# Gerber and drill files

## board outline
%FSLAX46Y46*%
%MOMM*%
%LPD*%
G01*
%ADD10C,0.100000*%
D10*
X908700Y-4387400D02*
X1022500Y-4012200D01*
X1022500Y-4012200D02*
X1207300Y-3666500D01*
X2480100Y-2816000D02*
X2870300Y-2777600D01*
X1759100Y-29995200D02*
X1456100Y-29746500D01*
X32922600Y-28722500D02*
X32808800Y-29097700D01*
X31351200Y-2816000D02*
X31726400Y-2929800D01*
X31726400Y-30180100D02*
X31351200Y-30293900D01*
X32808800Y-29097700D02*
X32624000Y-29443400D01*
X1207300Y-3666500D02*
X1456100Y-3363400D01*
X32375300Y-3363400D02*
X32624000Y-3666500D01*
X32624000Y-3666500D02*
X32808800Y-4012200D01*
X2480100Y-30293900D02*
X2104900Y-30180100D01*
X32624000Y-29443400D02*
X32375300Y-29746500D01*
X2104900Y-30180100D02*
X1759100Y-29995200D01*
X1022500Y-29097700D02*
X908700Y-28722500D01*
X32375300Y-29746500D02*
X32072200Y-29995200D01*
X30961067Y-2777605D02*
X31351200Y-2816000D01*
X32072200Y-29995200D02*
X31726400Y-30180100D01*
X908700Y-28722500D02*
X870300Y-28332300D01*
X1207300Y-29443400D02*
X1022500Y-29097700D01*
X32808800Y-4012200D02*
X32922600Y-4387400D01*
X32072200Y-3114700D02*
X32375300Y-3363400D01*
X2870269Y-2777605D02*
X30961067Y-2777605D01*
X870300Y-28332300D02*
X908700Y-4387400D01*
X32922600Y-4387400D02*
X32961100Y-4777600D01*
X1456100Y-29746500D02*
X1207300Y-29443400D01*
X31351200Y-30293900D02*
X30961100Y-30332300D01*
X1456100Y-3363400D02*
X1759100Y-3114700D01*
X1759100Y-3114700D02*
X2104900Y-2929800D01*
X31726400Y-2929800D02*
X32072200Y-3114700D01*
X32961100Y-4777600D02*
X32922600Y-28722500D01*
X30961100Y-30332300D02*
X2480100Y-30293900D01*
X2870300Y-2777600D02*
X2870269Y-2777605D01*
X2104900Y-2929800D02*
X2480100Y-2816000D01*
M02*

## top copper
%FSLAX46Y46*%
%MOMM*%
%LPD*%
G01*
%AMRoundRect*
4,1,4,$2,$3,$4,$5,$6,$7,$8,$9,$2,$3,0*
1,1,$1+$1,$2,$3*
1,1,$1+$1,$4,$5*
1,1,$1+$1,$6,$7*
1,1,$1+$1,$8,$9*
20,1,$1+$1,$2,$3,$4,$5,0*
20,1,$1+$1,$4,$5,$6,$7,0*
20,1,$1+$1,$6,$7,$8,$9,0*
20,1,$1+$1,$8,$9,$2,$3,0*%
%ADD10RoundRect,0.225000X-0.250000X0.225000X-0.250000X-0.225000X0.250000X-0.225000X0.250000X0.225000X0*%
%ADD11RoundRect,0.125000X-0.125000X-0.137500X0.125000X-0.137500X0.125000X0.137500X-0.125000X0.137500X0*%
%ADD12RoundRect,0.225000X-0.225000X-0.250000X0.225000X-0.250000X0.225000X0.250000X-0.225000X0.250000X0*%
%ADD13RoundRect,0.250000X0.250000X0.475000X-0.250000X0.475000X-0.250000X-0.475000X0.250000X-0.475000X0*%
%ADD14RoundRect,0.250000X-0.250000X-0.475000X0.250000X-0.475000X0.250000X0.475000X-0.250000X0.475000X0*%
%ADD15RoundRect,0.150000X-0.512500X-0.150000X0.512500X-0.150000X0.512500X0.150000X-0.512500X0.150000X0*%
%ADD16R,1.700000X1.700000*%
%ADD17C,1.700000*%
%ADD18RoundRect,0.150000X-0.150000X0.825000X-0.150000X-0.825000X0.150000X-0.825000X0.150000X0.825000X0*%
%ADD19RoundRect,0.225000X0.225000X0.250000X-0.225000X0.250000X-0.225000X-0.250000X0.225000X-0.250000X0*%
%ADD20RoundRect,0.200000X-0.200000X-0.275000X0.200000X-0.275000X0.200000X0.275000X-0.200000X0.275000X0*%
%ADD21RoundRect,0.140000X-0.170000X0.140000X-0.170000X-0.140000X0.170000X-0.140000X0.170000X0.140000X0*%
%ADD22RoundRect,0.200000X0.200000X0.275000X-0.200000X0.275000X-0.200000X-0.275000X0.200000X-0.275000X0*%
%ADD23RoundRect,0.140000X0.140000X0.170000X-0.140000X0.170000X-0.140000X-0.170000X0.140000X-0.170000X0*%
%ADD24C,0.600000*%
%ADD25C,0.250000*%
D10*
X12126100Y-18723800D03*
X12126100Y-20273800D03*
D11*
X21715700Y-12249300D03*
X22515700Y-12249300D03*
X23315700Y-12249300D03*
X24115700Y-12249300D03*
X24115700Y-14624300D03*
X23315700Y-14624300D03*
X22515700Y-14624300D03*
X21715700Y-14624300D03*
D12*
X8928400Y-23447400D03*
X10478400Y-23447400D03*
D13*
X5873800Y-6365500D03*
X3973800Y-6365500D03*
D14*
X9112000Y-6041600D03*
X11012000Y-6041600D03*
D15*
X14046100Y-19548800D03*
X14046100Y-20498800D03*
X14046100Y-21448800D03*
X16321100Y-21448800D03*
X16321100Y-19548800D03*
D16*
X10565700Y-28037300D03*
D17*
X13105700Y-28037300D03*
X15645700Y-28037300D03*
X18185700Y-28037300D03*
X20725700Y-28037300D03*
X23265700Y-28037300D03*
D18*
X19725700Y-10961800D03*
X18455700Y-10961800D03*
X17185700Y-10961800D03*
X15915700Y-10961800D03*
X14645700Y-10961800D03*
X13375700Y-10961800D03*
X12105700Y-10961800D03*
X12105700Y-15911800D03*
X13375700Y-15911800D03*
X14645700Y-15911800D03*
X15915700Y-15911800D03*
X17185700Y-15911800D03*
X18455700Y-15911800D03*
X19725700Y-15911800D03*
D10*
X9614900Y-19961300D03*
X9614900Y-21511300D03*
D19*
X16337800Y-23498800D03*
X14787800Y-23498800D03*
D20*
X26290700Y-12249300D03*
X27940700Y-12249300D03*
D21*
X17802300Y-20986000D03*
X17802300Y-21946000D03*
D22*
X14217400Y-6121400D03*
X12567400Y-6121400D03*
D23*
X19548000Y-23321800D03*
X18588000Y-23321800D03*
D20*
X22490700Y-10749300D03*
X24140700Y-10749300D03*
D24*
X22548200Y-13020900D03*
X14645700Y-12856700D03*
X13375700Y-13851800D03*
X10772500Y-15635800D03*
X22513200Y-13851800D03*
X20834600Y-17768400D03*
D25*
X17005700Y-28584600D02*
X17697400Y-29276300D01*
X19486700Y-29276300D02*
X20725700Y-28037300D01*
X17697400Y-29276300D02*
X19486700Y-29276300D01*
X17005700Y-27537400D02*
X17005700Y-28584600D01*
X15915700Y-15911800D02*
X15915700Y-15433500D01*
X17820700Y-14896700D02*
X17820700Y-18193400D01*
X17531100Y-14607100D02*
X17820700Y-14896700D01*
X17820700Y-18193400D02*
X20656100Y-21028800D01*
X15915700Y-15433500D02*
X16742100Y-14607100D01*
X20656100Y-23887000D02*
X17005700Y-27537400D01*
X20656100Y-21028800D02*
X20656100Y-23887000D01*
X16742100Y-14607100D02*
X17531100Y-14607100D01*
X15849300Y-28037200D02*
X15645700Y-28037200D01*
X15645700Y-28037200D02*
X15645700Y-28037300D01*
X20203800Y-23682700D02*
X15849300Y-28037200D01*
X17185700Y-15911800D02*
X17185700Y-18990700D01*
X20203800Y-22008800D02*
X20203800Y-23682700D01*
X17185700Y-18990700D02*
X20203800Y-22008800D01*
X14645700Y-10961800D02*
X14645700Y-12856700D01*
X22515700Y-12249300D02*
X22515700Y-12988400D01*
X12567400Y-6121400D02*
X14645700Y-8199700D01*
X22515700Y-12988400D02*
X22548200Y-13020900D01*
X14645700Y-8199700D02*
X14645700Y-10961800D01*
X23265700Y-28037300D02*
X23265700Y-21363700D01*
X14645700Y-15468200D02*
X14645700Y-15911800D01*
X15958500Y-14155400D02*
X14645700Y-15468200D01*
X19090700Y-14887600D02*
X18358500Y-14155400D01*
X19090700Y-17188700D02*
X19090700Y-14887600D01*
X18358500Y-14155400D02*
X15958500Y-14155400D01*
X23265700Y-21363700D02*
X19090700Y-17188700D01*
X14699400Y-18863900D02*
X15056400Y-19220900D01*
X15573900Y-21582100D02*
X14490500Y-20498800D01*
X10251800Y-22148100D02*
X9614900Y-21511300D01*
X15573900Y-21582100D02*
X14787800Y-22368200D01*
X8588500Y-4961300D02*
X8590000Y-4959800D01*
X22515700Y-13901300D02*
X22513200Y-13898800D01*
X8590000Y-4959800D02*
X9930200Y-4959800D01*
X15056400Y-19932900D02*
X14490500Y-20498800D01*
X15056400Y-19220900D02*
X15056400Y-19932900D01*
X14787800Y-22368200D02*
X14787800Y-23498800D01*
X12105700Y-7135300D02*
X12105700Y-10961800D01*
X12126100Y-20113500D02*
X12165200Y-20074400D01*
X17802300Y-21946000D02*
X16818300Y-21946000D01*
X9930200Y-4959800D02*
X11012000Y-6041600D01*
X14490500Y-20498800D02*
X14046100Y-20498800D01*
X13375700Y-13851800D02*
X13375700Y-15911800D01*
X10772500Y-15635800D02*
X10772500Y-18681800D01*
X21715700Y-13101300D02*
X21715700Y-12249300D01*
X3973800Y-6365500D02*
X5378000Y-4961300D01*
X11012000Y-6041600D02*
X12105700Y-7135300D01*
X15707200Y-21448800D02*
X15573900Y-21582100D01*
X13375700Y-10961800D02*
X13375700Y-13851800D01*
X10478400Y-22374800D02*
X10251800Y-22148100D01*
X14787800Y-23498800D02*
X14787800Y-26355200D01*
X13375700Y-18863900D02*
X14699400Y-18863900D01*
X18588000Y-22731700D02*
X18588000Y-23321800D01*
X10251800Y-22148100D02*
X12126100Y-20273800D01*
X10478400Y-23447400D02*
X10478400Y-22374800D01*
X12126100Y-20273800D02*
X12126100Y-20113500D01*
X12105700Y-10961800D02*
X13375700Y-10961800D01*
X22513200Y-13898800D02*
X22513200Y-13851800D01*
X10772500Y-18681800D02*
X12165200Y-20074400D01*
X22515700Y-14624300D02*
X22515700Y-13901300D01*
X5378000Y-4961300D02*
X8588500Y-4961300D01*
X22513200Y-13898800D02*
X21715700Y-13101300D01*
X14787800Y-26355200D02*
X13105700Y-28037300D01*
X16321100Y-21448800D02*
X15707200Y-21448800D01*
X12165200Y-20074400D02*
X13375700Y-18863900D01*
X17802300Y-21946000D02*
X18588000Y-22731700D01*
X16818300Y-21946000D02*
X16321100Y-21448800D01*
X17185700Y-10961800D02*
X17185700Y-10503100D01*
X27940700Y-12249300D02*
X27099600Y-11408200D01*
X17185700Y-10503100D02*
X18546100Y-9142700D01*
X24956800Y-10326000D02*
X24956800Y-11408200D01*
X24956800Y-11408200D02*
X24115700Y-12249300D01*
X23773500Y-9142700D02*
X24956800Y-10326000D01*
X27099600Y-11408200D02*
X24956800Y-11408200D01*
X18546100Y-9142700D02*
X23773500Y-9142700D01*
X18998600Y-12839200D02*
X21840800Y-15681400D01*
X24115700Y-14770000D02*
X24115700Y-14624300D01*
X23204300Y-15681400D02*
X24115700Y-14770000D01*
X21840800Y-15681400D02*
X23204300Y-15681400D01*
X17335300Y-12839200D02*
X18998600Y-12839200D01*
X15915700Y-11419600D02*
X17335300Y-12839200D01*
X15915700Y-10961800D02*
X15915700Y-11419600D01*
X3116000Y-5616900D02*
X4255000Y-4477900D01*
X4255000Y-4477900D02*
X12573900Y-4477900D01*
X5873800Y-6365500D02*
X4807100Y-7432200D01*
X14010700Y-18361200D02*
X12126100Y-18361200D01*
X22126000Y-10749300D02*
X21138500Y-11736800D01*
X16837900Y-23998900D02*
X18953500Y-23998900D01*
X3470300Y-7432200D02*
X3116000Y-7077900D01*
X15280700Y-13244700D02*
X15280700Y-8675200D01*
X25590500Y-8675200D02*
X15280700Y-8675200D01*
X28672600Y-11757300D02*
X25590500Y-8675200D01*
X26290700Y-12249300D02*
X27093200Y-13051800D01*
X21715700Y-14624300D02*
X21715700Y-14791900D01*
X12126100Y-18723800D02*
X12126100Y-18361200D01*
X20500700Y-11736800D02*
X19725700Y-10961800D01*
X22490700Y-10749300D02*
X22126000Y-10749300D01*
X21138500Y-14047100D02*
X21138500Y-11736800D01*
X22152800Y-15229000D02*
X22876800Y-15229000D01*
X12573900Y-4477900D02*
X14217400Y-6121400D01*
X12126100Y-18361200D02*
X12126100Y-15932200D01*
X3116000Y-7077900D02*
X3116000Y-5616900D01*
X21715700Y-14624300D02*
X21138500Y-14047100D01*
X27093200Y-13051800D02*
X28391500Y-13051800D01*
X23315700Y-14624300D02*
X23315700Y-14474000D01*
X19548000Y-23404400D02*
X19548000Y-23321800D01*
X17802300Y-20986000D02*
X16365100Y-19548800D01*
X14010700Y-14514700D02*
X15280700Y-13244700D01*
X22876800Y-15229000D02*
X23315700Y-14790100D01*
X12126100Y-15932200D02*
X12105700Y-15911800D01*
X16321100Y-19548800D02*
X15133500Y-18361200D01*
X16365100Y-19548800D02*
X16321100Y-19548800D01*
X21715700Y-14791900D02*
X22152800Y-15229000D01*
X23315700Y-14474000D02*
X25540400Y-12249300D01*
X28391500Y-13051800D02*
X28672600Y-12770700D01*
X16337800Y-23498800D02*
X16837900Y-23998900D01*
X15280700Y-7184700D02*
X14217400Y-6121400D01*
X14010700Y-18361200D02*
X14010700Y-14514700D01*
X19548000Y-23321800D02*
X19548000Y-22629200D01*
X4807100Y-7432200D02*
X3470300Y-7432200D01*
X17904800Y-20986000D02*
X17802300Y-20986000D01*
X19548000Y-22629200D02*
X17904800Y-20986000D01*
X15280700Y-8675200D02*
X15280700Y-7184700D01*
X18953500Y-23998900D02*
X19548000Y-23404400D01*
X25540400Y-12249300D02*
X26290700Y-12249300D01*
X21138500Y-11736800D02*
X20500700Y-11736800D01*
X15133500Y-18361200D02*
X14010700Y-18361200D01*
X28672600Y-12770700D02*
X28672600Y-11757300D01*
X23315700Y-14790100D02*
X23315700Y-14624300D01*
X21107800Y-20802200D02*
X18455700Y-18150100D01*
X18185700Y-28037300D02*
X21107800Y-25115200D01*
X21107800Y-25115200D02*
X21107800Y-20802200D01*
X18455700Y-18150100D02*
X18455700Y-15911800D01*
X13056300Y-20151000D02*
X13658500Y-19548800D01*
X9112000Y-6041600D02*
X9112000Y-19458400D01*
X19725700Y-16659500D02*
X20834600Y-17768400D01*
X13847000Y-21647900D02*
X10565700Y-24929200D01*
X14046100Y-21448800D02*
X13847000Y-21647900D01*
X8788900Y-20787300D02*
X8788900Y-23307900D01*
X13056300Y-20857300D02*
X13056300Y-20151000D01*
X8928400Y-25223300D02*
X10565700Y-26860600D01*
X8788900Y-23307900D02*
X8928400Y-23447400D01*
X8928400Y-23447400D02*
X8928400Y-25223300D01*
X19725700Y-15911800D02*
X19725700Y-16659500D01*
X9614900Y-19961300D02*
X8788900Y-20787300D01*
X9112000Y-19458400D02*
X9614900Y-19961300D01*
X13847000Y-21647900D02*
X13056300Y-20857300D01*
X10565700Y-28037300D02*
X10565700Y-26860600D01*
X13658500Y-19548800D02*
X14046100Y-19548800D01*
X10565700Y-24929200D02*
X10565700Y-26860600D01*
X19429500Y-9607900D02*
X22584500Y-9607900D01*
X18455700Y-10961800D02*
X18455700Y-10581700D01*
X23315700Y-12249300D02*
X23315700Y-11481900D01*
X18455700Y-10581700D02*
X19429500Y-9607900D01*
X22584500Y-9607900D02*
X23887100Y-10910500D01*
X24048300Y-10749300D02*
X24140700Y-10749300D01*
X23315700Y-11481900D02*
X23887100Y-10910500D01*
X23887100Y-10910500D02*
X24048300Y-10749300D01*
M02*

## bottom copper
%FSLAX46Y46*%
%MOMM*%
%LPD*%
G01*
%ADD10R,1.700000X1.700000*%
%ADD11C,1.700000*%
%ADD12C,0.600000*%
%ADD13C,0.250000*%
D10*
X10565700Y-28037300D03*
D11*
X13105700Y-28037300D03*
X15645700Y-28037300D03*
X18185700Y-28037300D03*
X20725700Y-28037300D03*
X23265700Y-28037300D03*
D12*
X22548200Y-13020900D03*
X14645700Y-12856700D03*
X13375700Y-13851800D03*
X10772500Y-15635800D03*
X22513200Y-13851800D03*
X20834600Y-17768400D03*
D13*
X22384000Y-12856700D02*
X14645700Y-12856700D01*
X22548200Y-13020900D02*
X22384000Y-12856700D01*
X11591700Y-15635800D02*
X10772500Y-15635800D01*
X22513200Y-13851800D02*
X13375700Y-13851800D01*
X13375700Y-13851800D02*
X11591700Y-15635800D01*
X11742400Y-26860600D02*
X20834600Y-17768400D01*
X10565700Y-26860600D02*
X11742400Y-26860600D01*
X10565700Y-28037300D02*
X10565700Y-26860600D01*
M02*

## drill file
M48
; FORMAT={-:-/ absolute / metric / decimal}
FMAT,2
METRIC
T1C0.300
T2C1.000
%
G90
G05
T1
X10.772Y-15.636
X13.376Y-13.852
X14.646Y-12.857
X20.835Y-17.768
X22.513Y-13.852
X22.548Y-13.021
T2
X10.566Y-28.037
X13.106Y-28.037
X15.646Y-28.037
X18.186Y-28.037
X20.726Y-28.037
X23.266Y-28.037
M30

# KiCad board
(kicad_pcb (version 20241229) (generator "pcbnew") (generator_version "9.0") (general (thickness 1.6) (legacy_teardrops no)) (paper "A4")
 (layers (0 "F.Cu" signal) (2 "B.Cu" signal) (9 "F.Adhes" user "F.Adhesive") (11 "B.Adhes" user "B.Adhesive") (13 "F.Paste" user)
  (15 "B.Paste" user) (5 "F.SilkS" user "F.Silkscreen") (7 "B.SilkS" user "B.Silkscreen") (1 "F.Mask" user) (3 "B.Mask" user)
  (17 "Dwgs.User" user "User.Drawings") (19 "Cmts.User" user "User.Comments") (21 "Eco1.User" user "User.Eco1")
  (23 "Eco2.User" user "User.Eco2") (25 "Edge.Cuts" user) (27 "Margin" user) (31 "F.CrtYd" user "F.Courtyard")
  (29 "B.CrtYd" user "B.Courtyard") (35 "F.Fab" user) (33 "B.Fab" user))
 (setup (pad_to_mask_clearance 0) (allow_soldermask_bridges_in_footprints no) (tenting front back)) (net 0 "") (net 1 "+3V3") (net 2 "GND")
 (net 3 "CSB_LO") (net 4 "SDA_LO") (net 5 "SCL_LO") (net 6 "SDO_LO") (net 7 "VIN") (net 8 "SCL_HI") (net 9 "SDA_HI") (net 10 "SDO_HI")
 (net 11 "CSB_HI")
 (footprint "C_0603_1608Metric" (layer "F.Cu") (at 12.1261 19.4988 -90)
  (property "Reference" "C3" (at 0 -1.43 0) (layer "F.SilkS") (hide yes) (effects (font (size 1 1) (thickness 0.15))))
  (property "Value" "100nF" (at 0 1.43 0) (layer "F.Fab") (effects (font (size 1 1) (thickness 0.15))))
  (pad "1" smd roundrect (at -0.775 0 270) (size 0.9 0.95) (layers "F.Cu" "F.Mask" "F.Paste") (roundrect_rratio 0.25) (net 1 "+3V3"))
  (pad "2" smd roundrect (at 0.775 0 270) (size 0.9 0.95) (layers "F.Cu" "F.Mask" "F.Paste") (roundrect_rratio 0.25) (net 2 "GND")))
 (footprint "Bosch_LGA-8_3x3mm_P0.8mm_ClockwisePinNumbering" (layer "F.Cu") (at 22.9157 13.4368)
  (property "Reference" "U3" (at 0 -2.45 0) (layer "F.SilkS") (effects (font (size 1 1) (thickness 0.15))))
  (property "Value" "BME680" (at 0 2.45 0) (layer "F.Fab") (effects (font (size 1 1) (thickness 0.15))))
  (pad "1" smd roundrect (at -1.2 -1.1875) (size 0.5 0.525) (layers "F.Cu" "F.Mask" "F.Paste") (roundrect_rratio 0.25) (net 2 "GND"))
  (pad "2" smd roundrect (at -0.4 -1.1875) (size 0.5 0.525) (layers "F.Cu" "F.Mask" "F.Paste") (roundrect_rratio 0.25) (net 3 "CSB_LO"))
  (pad "3" smd roundrect (at 0.4 -1.1875) (size 0.5 0.525) (layers "F.Cu" "F.Mask" "F.Paste") (roundrect_rratio 0.25) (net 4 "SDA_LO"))
  (pad "4" smd roundrect (at 1.2 -1.1875) (size 0.5 0.525) (layers "F.Cu" "F.Mask" "F.Paste") (roundrect_rratio 0.25) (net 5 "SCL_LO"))
  (pad "5" smd roundrect (at 1.2 1.1875) (size 0.5 0.525) (layers "F.Cu" "F.Mask" "F.Paste") (roundrect_rratio 0.25) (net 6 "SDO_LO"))
  (pad "6" smd roundrect (at 0.4 1.1875) (size 0.5 0.525) (layers "F.Cu" "F.Mask" "F.Paste") (roundrect_rratio 0.25) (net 1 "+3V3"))
  (pad "7" smd roundrect (at -0.4 1.1875) (size 0.5 0.525) (layers "F.Cu" "F.Mask" "F.Paste") (roundrect_rratio 0.25) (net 2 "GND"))
  (pad "8" smd roundrect (at -1.2 1.1875) (size 0.5 0.525) (layers "F.Cu" "F.Mask" "F.Paste") (roundrect_rratio 0.25) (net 1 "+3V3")))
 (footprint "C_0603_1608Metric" (layer "F.Cu") (at 9.7034 23.4474)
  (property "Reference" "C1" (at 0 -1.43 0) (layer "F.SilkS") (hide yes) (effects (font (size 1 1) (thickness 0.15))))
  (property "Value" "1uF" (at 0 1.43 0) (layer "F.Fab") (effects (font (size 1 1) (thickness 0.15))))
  (pad "1" smd roundrect (at -0.775 0) (size 0.9 0.95) (layers "F.Cu" "F.Mask" "F.Paste") (roundrect_rratio 0.25) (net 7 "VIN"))
  (pad "2" smd roundrect (at 0.775 0) (size 0.9 0.95) (layers "F.Cu" "F.Mask" "F.Paste") (roundrect_rratio 0.25) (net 2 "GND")))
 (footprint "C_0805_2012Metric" (layer "F.Cu") (at 4.9238 6.3655 180)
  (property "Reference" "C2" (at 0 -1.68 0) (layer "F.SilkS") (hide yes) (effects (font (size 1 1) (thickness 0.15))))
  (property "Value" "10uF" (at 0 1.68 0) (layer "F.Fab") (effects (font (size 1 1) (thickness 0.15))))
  (pad "1" smd roundrect (at -0.95 0 180) (size 1 1.45) (layers "F.Cu" "F.Mask" "F.Paste") (roundrect_rratio 0.25) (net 1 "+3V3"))
  (pad "2" smd roundrect (at 0.95 0 180) (size 1 1.45) (layers "F.Cu" "F.Mask" "F.Paste") (roundrect_rratio 0.25) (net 2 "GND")))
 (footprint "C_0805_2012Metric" (layer "F.Cu") (at 10.062 6.0416)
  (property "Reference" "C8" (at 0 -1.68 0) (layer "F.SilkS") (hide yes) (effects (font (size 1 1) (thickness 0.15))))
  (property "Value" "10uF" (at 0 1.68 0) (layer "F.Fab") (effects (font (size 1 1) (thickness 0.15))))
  (pad "1" smd roundrect (at -0.95 0) (size 1 1.45) (layers "F.Cu" "F.Mask" "F.Paste") (roundrect_rratio 0.25) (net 7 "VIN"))
  (pad "2" smd roundrect (at 0.95 0) (size 1 1.45) (layers "F.Cu" "F.Mask" "F.Paste") (roundrect_rratio 0.25) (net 2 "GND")))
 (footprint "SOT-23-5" (layer "F.Cu") (at 15.1836 20.4988)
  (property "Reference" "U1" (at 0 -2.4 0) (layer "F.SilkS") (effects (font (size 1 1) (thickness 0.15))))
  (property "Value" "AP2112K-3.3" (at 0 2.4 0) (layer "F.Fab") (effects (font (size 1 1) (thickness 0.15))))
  (pad "1" smd roundrect (at -1.1375 -0.95) (size 1.325 0.6) (layers "F.Cu" "F.Mask" "F.Paste") (roundrect_rratio 0.25) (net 7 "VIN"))
  (pad "2" smd roundrect (at -1.1375 0) (size 1.325 0.6) (layers "F.Cu" "F.Mask" "F.Paste") (roundrect_rratio 0.25) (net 2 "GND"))
  (pad "3" smd roundrect (at -1.1375 0.95) (size 1.325 0.6) (layers "F.Cu" "F.Mask" "F.Paste") (roundrect_rratio 0.25) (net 7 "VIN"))
  (pad "4" smd roundrect (at 1.1375 0.95) (size 1.325 0.6) (layers "F.Cu" "F.Mask" "F.Paste") (roundrect_rratio 0.25) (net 2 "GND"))
  (pad "5" smd roundrect (at 1.1375 -0.95) (size 1.325 0.6) (layers "F.Cu" "F.Mask" "F.Paste") (roundrect_rratio 0.25) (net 1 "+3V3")))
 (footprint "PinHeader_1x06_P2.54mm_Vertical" (layer "F.Cu") (at 10.5657 28.0373 90)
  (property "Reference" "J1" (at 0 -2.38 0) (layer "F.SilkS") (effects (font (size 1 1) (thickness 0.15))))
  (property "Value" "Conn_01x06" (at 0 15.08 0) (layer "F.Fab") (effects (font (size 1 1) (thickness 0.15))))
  (pad "1" thru_hole rect (at 0 0 90) (size 1.7 1.7) (drill 1) (layers "*.Cu" "*.Mask") (remove_unused_layers no) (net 7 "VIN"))
  (pad "2" thru_hole circle (at 0 2.54 90) (size 1.7 1.7) (drill 1) (layers "*.Cu" "*.Mask") (remove_unused_layers no) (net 2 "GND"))
  (pad "3" thru_hole circle (at 0 5.08 90) (size 1.7 1.7) (drill 1) (layers "*.Cu" "*.Mask") (remove_unused_layers no) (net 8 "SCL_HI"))
  (pad "4" thru_hole circle (at 0 7.62 90) (size 1.7 1.7) (drill 1) (layers "*.Cu" "*.Mask") (remove_unused_layers no) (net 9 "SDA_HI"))
  (pad "5" thru_hole circle (at 0 10.16 90) (size 1.7 1.7) (drill 1) (layers "*.Cu" "*.Mask") (remove_unused_layers no) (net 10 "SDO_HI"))
  (pad "6" thru_hole circle (at 0 12.7 90) (size 1.7 1.7) (drill 1) (layers "*.Cu" "*.Mask") (remove_unused_layers no) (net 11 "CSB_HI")))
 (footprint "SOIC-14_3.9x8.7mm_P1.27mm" (layer "F.Cu") (at 15.9157 13.4368 -90)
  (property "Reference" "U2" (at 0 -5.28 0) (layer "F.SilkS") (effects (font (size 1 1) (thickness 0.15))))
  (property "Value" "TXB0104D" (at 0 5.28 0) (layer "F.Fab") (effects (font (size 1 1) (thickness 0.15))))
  (pad "1" smd roundrect (at -2.475 -3.81 270) (size 1.95 0.6) (layers "F.Cu" "F.Mask" "F.Paste") (roundrect_rratio 0.25) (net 1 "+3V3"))
  (pad "2" smd roundrect (at -2.475 -2.54 270) (size 1.95 0.6) (layers "F.Cu" "F.Mask" "F.Paste") (roundrect_rratio 0.25) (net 4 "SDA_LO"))
  (pad "3" smd roundrect (at -2.475 -1.27 270) (size 1.95 0.6) (layers "F.Cu" "F.Mask" "F.Paste") (roundrect_rratio 0.25) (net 5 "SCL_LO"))
  (pad "4" smd roundrect (at -2.475 0 270) (size 1.95 0.6) (layers "F.Cu" "F.Mask" "F.Paste") (roundrect_rratio 0.25) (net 6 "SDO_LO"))
  (pad "5" smd roundrect (at -2.475 1.27 270) (size 1.95 0.6) (layers "F.Cu" "F.Mask" "F.Paste") (roundrect_rratio 0.25) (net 3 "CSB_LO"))
  (pad "6" smd roundrect (at -2.475 2.54 270) (size 1.95 0.6) (layers "F.Cu" "F.Mask" "F.Paste") (roundrect_rratio 0.25) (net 2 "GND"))
  (pad "7" smd roundrect (at -2.475 3.81 270) (size 1.95 0.6) (layers "F.Cu" "F.Mask" "F.Paste") (roundrect_rratio 0.25) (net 2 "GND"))
  (pad "8" smd roundrect (at 2.475 3.81 270) (size 1.95 0.6) (layers "F.Cu" "F.Mask" "F.Paste") (roundrect_rratio 0.25) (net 1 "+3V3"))
  (pad "9" smd roundrect (at 2.475 2.54 270) (size 1.95 0.6) (layers "F.Cu" "F.Mask" "F.Paste") (roundrect_rratio 0.25) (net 2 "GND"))
  (pad "10" smd roundrect (at 2.475 1.27 270) (size 1.95 0.6) (layers "F.Cu" "F.Mask" "F.Paste") (roundrect_rratio 0.25) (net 11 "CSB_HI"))
  (pad "11" smd roundrect (at 2.475 0 270) (size 1.95 0.6) (layers "F.Cu" "F.Mask" "F.Paste") (roundrect_rratio 0.25) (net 10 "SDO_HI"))
  (pad "12" smd roundrect (at 2.475 -1.27 270) (size 1.95 0.6) (layers "F.Cu" "F.Mask" "F.Paste") (roundrect_rratio 0.25) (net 8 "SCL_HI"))
  (pad "13" smd roundrect (at 2.475 -2.54 270) (size 1.95 0.6) (layers "F.Cu" "F.Mask" "F.Paste") (roundrect_rratio 0.25) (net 9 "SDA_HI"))
  (pad "14" smd roundrect (at 2.475 -3.81 270) (size 1.95 0.6) (layers "F.Cu" "F.Mask" "F.Paste") (roundrect_rratio 0.25) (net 7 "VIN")))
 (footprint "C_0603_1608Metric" (layer "F.Cu") (at 9.6149 20.7363 -90)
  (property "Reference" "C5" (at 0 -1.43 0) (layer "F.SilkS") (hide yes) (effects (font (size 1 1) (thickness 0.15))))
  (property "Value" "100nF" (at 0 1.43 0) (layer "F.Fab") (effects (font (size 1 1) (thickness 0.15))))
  (pad "1" smd roundrect (at -0.775 0 270) (size 0.9 0.95) (layers "F.Cu" "F.Mask" "F.Paste") (roundrect_rratio 0.25) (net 7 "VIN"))
  (pad "2" smd roundrect (at 0.775 0 270) (size 0.9 0.95) (layers "F.Cu" "F.Mask" "F.Paste") (roundrect_rratio 0.25) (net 2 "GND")))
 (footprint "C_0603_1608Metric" (layer "F.Cu") (at 15.5628 23.4988 180)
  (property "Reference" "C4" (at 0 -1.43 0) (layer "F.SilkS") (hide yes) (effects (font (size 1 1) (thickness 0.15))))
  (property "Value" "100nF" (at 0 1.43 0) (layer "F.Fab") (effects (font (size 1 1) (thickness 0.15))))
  (pad "1" smd roundrect (at -0.775 0 180) (size 0.9 0.95) (layers "F.Cu" "F.Mask" "F.Paste") (roundrect_rratio 0.25) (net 1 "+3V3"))
  (pad "2" smd roundrect (at 0.775 0 180) (size 0.9 0.95) (layers "F.Cu" "F.Mask" "F.Paste") (roundrect_rratio 0.25) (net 2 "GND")))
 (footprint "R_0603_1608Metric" (layer "F.Cu") (at 27.1157 12.2493)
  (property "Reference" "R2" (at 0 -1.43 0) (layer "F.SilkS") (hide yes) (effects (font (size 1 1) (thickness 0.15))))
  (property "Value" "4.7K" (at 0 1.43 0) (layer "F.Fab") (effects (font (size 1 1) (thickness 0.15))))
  (pad "1" smd roundrect (at -0.825 0) (size 0.8 0.95) (layers "F.Cu" "F.Mask" "F.Paste") (roundrect_rratio 0.25) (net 1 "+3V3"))
  (pad "2" smd roundrect (at 0.825 0) (size 0.8 0.95) (layers "F.Cu" "F.Mask" "F.Paste") (roundrect_rratio 0.25) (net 5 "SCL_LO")))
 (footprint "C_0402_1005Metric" (layer "F.Cu") (at 17.8023 21.466 -90)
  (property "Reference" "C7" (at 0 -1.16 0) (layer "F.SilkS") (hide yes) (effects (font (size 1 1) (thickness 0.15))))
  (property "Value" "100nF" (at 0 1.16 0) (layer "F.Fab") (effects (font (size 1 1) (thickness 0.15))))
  (pad "1" smd roundrect (at -0.48 0 270) (size 0.56 0.62) (layers "F.Cu" "F.Mask" "F.Paste") (roundrect_rratio 0.25) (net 1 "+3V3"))
  (pad "2" smd roundrect (at 0.48 0 270) (size 0.56 0.62) (layers "F.Cu" "F.Mask" "F.Paste") (roundrect_rratio 0.25) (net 2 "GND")))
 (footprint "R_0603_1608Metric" (layer "F.Cu") (at 13.3924 6.1214 180)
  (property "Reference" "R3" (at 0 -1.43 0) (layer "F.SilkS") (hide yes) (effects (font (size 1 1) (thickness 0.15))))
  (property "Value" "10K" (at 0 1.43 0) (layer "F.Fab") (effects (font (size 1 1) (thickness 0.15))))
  (pad "1" smd roundrect (at -0.825 0 180) (size 0.8 0.95) (layers "F.Cu" "F.Mask" "F.Paste") (roundrect_rratio 0.25) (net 1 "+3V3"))
  (pad "2" smd roundrect (at 0.825 0 180) (size 0.8 0.95) (layers "F.Cu" "F.Mask" "F.Paste") (roundrect_rratio 0.25) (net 3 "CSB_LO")))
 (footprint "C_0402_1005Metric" (layer "F.Cu") (at 19.068 23.3218 180)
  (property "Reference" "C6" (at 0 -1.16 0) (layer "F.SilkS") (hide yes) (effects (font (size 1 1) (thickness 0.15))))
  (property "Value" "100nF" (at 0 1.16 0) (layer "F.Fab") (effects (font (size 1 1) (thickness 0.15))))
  (pad "1" smd roundrect (at -0.48 0 180) (size 0.56 0.62) (layers "F.Cu" "F.Mask" "F.Paste") (roundrect_rratio 0.25) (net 1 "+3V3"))
  (pad "2" smd roundrect (at 0.48 0 180) (size 0.56 0.62) (layers "F.Cu" "F.Mask" "F.Paste") (roundrect_rratio 0.25) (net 2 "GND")))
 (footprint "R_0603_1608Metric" (layer "F.Cu") (at 23.3157 10.7493)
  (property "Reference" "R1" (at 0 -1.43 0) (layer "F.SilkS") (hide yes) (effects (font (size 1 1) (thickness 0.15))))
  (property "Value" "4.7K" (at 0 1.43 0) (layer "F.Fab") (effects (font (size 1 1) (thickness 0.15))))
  (pad "1" smd roundrect (at -0.825 0) (size 0.8 0.95) (layers "F.Cu" "F.Mask" "F.Paste") (roundrect_rratio 0.25) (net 1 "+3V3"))
  (pad "2" smd roundrect (at 0.825 0) (size 0.8 0.95) (layers "F.Cu" "F.Mask" "F.Paste") (roundrect_rratio 0.25) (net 4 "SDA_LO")))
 (gr_line (start 0.9087 4.3874) (end 1.0225 4.0122) (stroke (width 0.1) (type solid)) (layer "Edge.Cuts"))
 (gr_line (start 1.0225 4.0122) (end 1.2073 3.6665) (stroke (width 0.1) (type solid)) (layer "Edge.Cuts"))
 (gr_line (start 2.4801 2.816) (end 2.8703 2.7776) (stroke (width 0.1) (type solid)) (layer "Edge.Cuts"))
 (gr_line (start 1.7591 29.9952) (end 1.4561 29.7465) (stroke (width 0.1) (type solid)) (layer "Edge.Cuts"))
 (gr_line (start 32.9226 28.7225) (end 32.8088 29.0977) (stroke (width 0.1) (type solid)) (layer "Edge.Cuts"))
 (gr_line (start 31.3512 2.816) (end 31.7264 2.9298) (stroke (width 0.1) (type solid)) (layer "Edge.Cuts"))
 (gr_line (start 31.7264 30.1801) (end 31.3512 30.2939) (stroke (width 0.1) (type solid)) (layer "Edge.Cuts"))
 (gr_line (start 32.8088 29.0977) (end 32.624 29.4434) (stroke (width 0.1) (type solid)) (layer "Edge.Cuts"))
 (gr_line (start 1.2073 3.6665) (end 1.4561 3.3634) (stroke (width 0.1) (type solid)) (layer "Edge.Cuts"))
 (gr_line (start 32.3753 3.3634) (end 32.624 3.6665) (stroke (width 0.1) (type solid)) (layer "Edge.Cuts"))
 (gr_line (start 32.624 3.6665) (end 32.8088 4.0122) (stroke (width 0.1) (type solid)) (layer "Edge.Cuts"))
 (gr_line (start 2.4801 30.2939) (end 2.1049 30.1801) (stroke (width 0.1) (type solid)) (layer "Edge.Cuts"))
 (gr_line (start 32.624 29.4434) (end 32.3753 29.7465) (stroke (width 0.1) (type solid)) (layer "Edge.Cuts"))
 (gr_line (start 2.1049 30.1801) (end 1.7591 29.9952) (stroke (width 0.1) (type solid)) (layer "Edge.Cuts"))
 (gr_line (start 1.0225 29.0977) (end 0.9087 28.7225) (stroke (width 0.1) (type solid)) (layer "Edge.Cuts"))
 (gr_line (start 32.3753 29.7465) (end 32.0722 29.9952) (stroke (width 0.1) (type solid)) (layer "Edge.Cuts"))
 (gr_line (start 30.961067 2.777605) (end 31.3512 2.816) (stroke (width 0.1) (type solid)) (layer "Edge.Cuts"))
 (gr_line (start 32.0722 29.9952) (end 31.7264 30.1801) (stroke (width 0.1) (type solid)) (layer "Edge.Cuts"))
 (gr_line (start 0.9087 28.7225) (end 0.8703 28.3323) (stroke (width 0.1) (type solid)) (layer "Edge.Cuts"))
 (gr_line (start 1.2073 29.4434) (end 1.0225 29.0977) (stroke (width 0.1) (type solid)) (layer "Edge.Cuts"))
 (gr_line (start 32.8088 4.0122) (end 32.9226 4.3874) (stroke (width 0.1) (type solid)) (layer "Edge.Cuts"))
 (gr_line (start 32.0722 3.1147) (end 32.3753 3.3634) (stroke (width 0.1) (type solid)) (layer "Edge.Cuts"))
 (gr_line (start 2.870269 2.777605) (end 30.961067 2.777605) (stroke (width 0.1) (type solid)) (layer "Edge.Cuts"))
 (gr_line (start 0.8703 28.3323) (end 0.9087 4.3874) (stroke (width 0.1) (type solid)) (layer "Edge.Cuts"))
 (gr_line (start 32.9226 4.3874) (end 32.9611 4.7776) (stroke (width 0.1) (type solid)) (layer "Edge.Cuts"))
 (gr_line (start 1.4561 29.7465) (end 1.2073 29.4434) (stroke (width 0.1) (type solid)) (layer "Edge.Cuts"))
 (gr_line (start 31.3512 30.2939) (end 30.9611 30.3323) (stroke (width 0.1) (type solid)) (layer "Edge.Cuts"))
 (gr_line (start 1.4561 3.3634) (end 1.7591 3.1147) (stroke (width 0.1) (type solid)) (layer "Edge.Cuts"))
 (gr_line (start 1.7591 3.1147) (end 2.1049 2.9298) (stroke (width 0.1) (type solid)) (layer "Edge.Cuts"))
 (gr_line (start 31.7264 2.9298) (end 32.0722 3.1147) (stroke (width 0.1) (type solid)) (layer "Edge.Cuts"))
 (gr_line (start 32.9611 4.7776) (end 32.9226 28.7225) (stroke (width 0.1) (type solid)) (layer "Edge.Cuts"))
 (gr_line (start 30.9611 30.3323) (end 2.4801 30.2939) (stroke (width 0.1) (type solid)) (layer "Edge.Cuts"))
 (gr_line (start 2.8703 2.7776) (end 2.870269 2.777605) (stroke (width 0.1) (type solid)) (layer "Edge.Cuts"))
 (gr_line (start 2.1049 2.9298) (end 2.4801 2.816) (stroke (width 0.1) (type solid)) (layer "Edge.Cuts"))
 (segment (start 17.0057 28.5846) (end 17.6974 29.2763) (width 0.25) (layer "F.Cu") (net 10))
 (segment (start 19.4867 29.2763) (end 20.7257 28.0373) (width 0.25) (layer "F.Cu") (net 10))
 (segment (start 17.6974 29.2763) (end 19.4867 29.2763) (width 0.25) (layer "F.Cu") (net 10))
 (segment (start 17.0057 27.5374) (end 17.0057 28.5846) (width 0.25) (layer "F.Cu") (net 10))
 (segment (start 15.9157 15.9118) (end 15.9157 15.4335) (width 0.25) (layer "F.Cu") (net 10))
 (segment (start 17.8207 14.8967) (end 17.8207 18.1934) (width 0.25) (layer "F.Cu") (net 10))
 (segment (start 17.5311 14.6071) (end 17.8207 14.8967) (width 0.25) (layer "F.Cu") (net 10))
 (segment (start 17.8207 18.1934) (end 20.6561 21.0288) (width 0.25) (layer "F.Cu") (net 10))
 (segment (start 15.9157 15.4335) (end 16.7421 14.6071) (width 0.25) (layer "F.Cu") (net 10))
 (segment (start 20.6561 23.887) (end 17.0057 27.5374) (width 0.25) (layer "F.Cu") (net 10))
 (segment (start 20.6561 21.0288) (end 20.6561 23.887) (width 0.25) (layer "F.Cu") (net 10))
 (segment (start 16.7421 14.6071) (end 17.5311 14.6071) (width 0.25) (layer "F.Cu") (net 10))
 (segment (start 15.8493 28.0372) (end 15.6457 28.0372) (width 0.25) (layer "F.Cu") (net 8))
 (segment (start 15.6457 28.0372) (end 15.6457 28.0373) (width 0.25) (layer "F.Cu") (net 8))
 (segment (start 20.2038 23.6827) (end 15.8493 28.0372) (width 0.25) (layer "F.Cu") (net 8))
 (segment (start 17.1857 15.9118) (end 17.1857 18.9907) (width 0.25) (layer "F.Cu") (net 8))
 (segment (start 20.2038 22.0088) (end 20.2038 23.6827) (width 0.25) (layer "F.Cu") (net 8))
 (segment (start 17.1857 18.9907) (end 20.2038 22.0088) (width 0.25) (layer "F.Cu") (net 8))
 (segment (start 14.6457 10.9618) (end 14.6457 12.8567) (width 0.25) (layer "F.Cu") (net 3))
 (segment (start 22.5157 12.2493) (end 22.5157 12.9884) (width 0.25) (layer "F.Cu") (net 3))
 (segment (start 12.5674 6.1214) (end 14.6457 8.1997) (width 0.25) (layer "F.Cu") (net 3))
 (segment (start 22.5157 12.9884) (end 22.5482 13.0209) (width 0.25) (layer "F.Cu") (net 3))
 (segment (start 14.6457 8.1997) (end 14.6457 10.9618) (width 0.25) (layer "F.Cu") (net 3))
 (via (at 22.5482 13.0209) (size 0.6) (drill 0.3) (layers "F.Cu" "B.Cu") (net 3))
 (via (at 14.6457 12.8567) (size 0.6) (drill 0.3) (layers "F.Cu" "B.Cu") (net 3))
 (segment (start 22.384 12.8567) (end 14.6457 12.8567) (width 0.25) (layer "B.Cu") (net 3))
 (segment (start 22.5482 13.0209) (end 22.384 12.8567) (width 0.25) (layer "B.Cu") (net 3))
 (segment (start 23.2657 28.0373) (end 23.2657 21.3637) (width 0.25) (layer "F.Cu") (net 11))
 (segment (start 14.6457 15.4682) (end 14.6457 15.9118) (width 0.25) (layer "F.Cu") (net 11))
 (segment (start 15.9585 14.1554) (end 14.6457 15.4682) (width 0.25) (layer "F.Cu") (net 11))
 (segment (start 19.0907 14.8876) (end 18.3585 14.1554) (width 0.25) (layer "F.Cu") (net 11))
 (segment (start 19.0907 17.1887) (end 19.0907 14.8876) (width 0.25) (layer "F.Cu") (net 11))
 (segment (start 18.3585 14.1554) (end 15.9585 14.1554) (width 0.25) (layer "F.Cu") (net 11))
 (segment (start 23.2657 21.3637) (end 19.0907 17.1887) (width 0.25) (layer "F.Cu") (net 11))
 (segment (start 14.6994 18.8639) (end 15.0564 19.2209) (width 0.25) (layer "F.Cu") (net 2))
 (segment (start 15.5739 21.5821) (end 14.4905 20.4988) (width 0.25) (layer "F.Cu") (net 2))
 (segment (start 10.2518 22.1481) (end 9.6149 21.5113) (width 0.25) (layer "F.Cu") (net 2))
 (segment (start 15.5739 21.5821) (end 14.7878 22.3682) (width 0.25) (layer "F.Cu") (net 2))
 (segment (start 8.5885 4.9613) (end 8.59 4.9598) (width 0.25) (layer "F.Cu") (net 2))
 (segment (start 22.5157 13.9013) (end 22.5132 13.8988) (width 0.25) (layer "F.Cu") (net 2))
 (segment (start 8.59 4.9598) (end 9.9302 4.9598) (width 0.25) (layer "F.Cu") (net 2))
 (segment (start 15.0564 19.9329) (end 14.4905 20.4988) (width 0.25) (layer "F.Cu") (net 2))
 (segment (start 15.0564 19.2209) (end 15.0564 19.9329) (width 0.25) (layer "F.Cu") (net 2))
 (segment (start 14.7878 22.3682) (end 14.7878 23.4988) (width 0.25) (layer "F.Cu") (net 2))
 (segment (start 12.1057 7.1353) (end 12.1057 10.9618) (width 0.25) (layer "F.Cu") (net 2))
 (segment (start 12.1261 20.1135) (end 12.1652 20.0744) (width 0.25) (layer "F.Cu") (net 2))
 (segment (start 17.8023 21.946) (end 16.8183 21.946) (width 0.25) (layer "F.Cu") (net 2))
 (segment (start 9.9302 4.9598) (end 11.012 6.0416) (width 0.25) (layer "F.Cu") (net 2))
 (segment (start 14.4905 20.4988) (end 14.0461 20.4988) (width 0.25) (layer "F.Cu") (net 2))
 (segment (start 13.3757 13.8518) (end 13.3757 15.9118) (width 0.25) (layer "F.Cu") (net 2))
 (segment (start 10.7725 15.6358) (end 10.7725 18.6818) (width 0.25) (layer "F.Cu") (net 2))
 (segment (start 21.7157 13.1013) (end 21.7157 12.2493) (width 0.25) (layer "F.Cu") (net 2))
 (segment (start 3.9738 6.3655) (end 5.378 4.9613) (width 0.25) (layer "F.Cu") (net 2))
 (segment (start 11.012 6.0416) (end 12.1057 7.1353) (width 0.25) (layer "F.Cu") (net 2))
 (segment (start 15.7072 21.4488) (end 15.5739 21.5821) (width 0.25) (layer "F.Cu") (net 2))
 (segment (start 13.3757 10.9618) (end 13.3757 13.8518) (width 0.25) (layer "F.Cu") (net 2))
 (segment (start 10.4784 22.3748) (end 10.2518 22.1481) (width 0.25) (layer "F.Cu") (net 2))
 (segment (start 14.7878 23.4988) (end 14.7878 26.3552) (width 0.25) (layer "F.Cu") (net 2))
 (segment (start 13.3757 18.8639) (end 14.6994 18.8639) (width 0.25) (layer "F.Cu") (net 2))
 (segment (start 18.588 22.7317) (end 18.588 23.3218) (width 0.25) (layer "F.Cu") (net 2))
 (segment (start 10.2518 22.1481) (end 12.1261 20.2738) (width 0.25) (layer "F.Cu") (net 2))
 (segment (start 10.4784 23.4474) (end 10.4784 22.3748) (width 0.25) (layer "F.Cu") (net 2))
 (segment (start 12.1261 20.2738) (end 12.1261 20.1135) (width 0.25) (layer "F.Cu") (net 2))
 (segment (start 12.1057 10.9618) (end 13.3757 10.9618) (width 0.25) (layer "F.Cu") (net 2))
 (segment (start 22.5132 13.8988) (end 22.5132 13.8518) (width 0.25) (layer "F.Cu") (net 2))
 (segment (start 10.7725 18.6818) (end 12.1652 20.0744) (width 0.25) (layer "F.Cu") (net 2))
 (segment (start 22.5157 14.6243) (end 22.5157 13.9013) (width 0.25) (layer "F.Cu") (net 2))
 (segment (start 5.378 4.9613) (end 8.5885 4.9613) (width 0.25) (layer "F.Cu") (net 2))
 (segment (start 22.5132 13.8988) (end 21.7157 13.1013) (width 0.25) (layer "F.Cu") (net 2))
 (segment (start 14.7878 26.3552) (end 13.1057 28.0373) (width 0.25) (layer "F.Cu") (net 2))
 (segment (start 16.3211 21.4488) (end 15.7072 21.4488) (width 0.25) (layer "F.Cu") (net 2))
 (segment (start 12.1652 20.0744) (end 13.3757 18.8639) (width 0.25) (layer "F.Cu") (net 2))
 (segment (start 17.8023 21.946) (end 18.588 22.7317) (width 0.25) (layer "F.Cu") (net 2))
 (segment (start 16.8183 21.946) (end 16.3211 21.4488) (width 0.25) (layer "F.Cu") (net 2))
 (via (at 13.3757 13.8518) (size 0.6) (drill 0.3) (layers "F.Cu" "B.Cu") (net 2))
 (via (at 10.7725 15.6358) (size 0.6) (drill 0.3) (layers "F.Cu" "B.Cu") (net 2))
 (via (at 22.5132 13.8518) (size 0.6) (drill 0.3) (layers "F.Cu" "B.Cu") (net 2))
 (segment (start 11.5917 15.6358) (end 10.7725 15.6358) (width 0.25) (layer "B.Cu") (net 2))
 (segment (start 22.5132 13.8518) (end 13.3757 13.8518) (width 0.25) (layer "B.Cu") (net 2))
 (segment (start 13.3757 13.8518) (end 11.5917 15.6358) (width 0.25) (layer "B.Cu") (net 2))
 (segment (start 17.1857 10.9618) (end 17.1857 10.5031) (width 0.25) (layer "F.Cu") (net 5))
 (segment (start 27.9407 12.2493) (end 27.0996 11.4082) (width 0.25) (layer "F.Cu") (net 5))
 (segment (start 17.1857 10.5031) (end 18.5461 9.1427) (width 0.25) (layer "F.Cu") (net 5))
 (segment (start 24.9568 10.326) (end 24.9568 11.4082) (width 0.25) (layer "F.Cu") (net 5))
 (segment (start 24.9568 11.4082) (end 24.1157 12.2493) (width 0.25) (layer "F.Cu") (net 5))
 (segment (start 23.7735 9.1427) (end 24.9568 10.326) (width 0.25) (layer "F.Cu") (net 5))
 (segment (start 27.0996 11.4082) (end 24.9568 11.4082) (width 0.25) (layer "F.Cu") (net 5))
 (segment (start 18.5461 9.1427) (end 23.7735 9.1427) (width 0.25) (layer "F.Cu") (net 5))
 (segment (start 18.9986 12.8392) (end 21.8408 15.6814) (width 0.25) (layer "F.Cu") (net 6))
 (segment (start 24.1157 14.77) (end 24.1157 14.6243) (width 0.25) (layer "F.Cu") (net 6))
 (segment (start 23.2043 15.6814) (end 24.1157 14.77) (width 0.25) (layer "F.Cu") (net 6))
 (segment (start 21.8408 15.6814) (end 23.2043 15.6814) (width 0.25) (layer "F.Cu") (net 6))
 (segment (start 17.3353 12.8392) (end 18.9986 12.8392) (width 0.25) (layer "F.Cu") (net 6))
 (segment (start 15.9157 11.4196) (end 17.3353 12.8392) (width 0.25) (layer "F.Cu") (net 6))
 (segment (start 15.9157 10.9618) (end 15.9157 11.4196) (width 0.25) (layer "F.Cu") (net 6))
 (segment (start 3.116 5.6169) (end 4.255 4.4779) (width 0.25) (layer "F.Cu") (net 1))
 (segment (start 4.255 4.4779) (end 12.5739 4.4779) (width 0.25) (layer "F.Cu") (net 1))
 (segment (start 5.8738 6.3655) (end 4.8071 7.4322) (width 0.25) (layer "F.Cu") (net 1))
 (segment (start 14.0107 18.3612) (end 12.1261 18.3612) (width 0.25) (layer "F.Cu") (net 1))
 (segment (start 22.126 10.7493) (end 21.1385 11.7368) (width 0.25) (layer "F.Cu") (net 1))
 (segment (start 16.8379 23.9989) (end 18.9535 23.9989) (width 0.25) (layer "F.Cu") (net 1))
 (segment (start 3.4703 7.4322) (end 3.116 7.0779) (width 0.25) (layer "F.Cu") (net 1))
 (segment (start 15.2807 13.2447) (end 15.2807 8.6752) (width 0.25) (layer "F.Cu") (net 1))
 (segment (start 25.5905 8.6752) (end 15.2807 8.6752) (width 0.25) (layer "F.Cu") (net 1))
 (segment (start 28.6726 11.7573) (end 25.5905 8.6752) (width 0.25) (layer "F.Cu") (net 1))
 (segment (start 26.2907 12.2493) (end 27.0932 13.0518) (width 0.25) (layer "F.Cu") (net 1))
 (segment (start 21.7157 14.6243) (end 21.7157 14.7919) (width 0.25) (layer "F.Cu") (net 1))
 (segment (start 12.1261 18.7238) (end 12.1261 18.3612) (width 0.25) (layer "F.Cu") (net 1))
 (segment (start 20.5007 11.7368) (end 19.7257 10.9618) (width 0.25) (layer "F.Cu") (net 1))
 (segment (start 22.4907 10.7493) (end 22.126 10.7493) (width 0.25) (layer "F.Cu") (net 1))
 (segment (start 21.1385 14.0471) (end 21.1385 11.7368) (width 0.25) (layer "F.Cu") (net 1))
 (segment (start 22.1528 15.229) (end 22.8768 15.229) (width 0.25) (layer "F.Cu") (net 1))
 (segment (start 12.5739 4.4779) (end 14.2174 6.1214) (width 0.25) (layer "F.Cu") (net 1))
 (segment (start 12.1261 18.3612) (end 12.1261 15.9322) (width 0.25) (layer "F.Cu") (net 1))
 (segment (start 3.116 7.0779) (end 3.116 5.6169) (width 0.25) (layer "F.Cu") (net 1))
 (segment (start 21.7157 14.6243) (end 21.1385 14.0471) (width 0.25) (layer "F.Cu") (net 1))
 (segment (start 27.0932 13.0518) (end 28.3915 13.0518) (width 0.25) (layer "F.Cu") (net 1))
 (segment (start 23.3157 14.6243) (end 23.3157 14.474) (width 0.25) (layer "F.Cu") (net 1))
 (segment (start 19.548 23.4044) (end 19.548 23.3218) (width 0.25) (layer "F.Cu") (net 1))
 (segment (start 17.8023 20.986) (end 16.3651 19.5488) (width 0.25) (layer "F.Cu") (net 1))
 (segment (start 14.0107 14.5147) (end 15.2807 13.2447) (width 0.25) (layer "F.Cu") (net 1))
 (segment (start 22.8768 15.229) (end 23.3157 14.7901) (width 0.25) (layer "F.Cu") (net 1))
 (segment (start 12.1261 15.9322) (end 12.1057 15.9118) (width 0.25) (layer "F.Cu") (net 1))
 (segment (start 16.3211 19.5488) (end 15.1335 18.3612) (width 0.25) (layer "F.Cu") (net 1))
 (segment (start 16.3651 19.5488) (end 16.3211 19.5488) (width 0.25) (layer "F.Cu") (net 1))
 (segment (start 21.7157 14.7919) (end 22.1528 15.229) (width 0.25) (layer "F.Cu") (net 1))
 (segment (start 23.3157 14.474) (end 25.5404 12.2493) (width 0.25) (layer "F.Cu") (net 1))
 (segment (start 28.3915 13.0518) (end 28.6726 12.7707) (width 0.25) (layer "F.Cu") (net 1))
 (segment (start 16.3378 23.4988) (end 16.8379 23.9989) (width 0.25) (layer "F.Cu") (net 1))
 (segment (start 15.2807 7.1847) (end 14.2174 6.1214) (width 0.25) (layer "F.Cu") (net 1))
 (segment (start 14.0107 18.3612) (end 14.0107 14.5147) (width 0.25) (layer "F.Cu") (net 1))
 (segment (start 19.548 23.3218) (end 19.548 22.6292) (width 0.25) (layer "F.Cu") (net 1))
 (segment (start 4.8071 7.4322) (end 3.4703 7.4322) (width 0.25) (layer "F.Cu") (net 1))
 (segment (start 17.9048 20.986) (end 17.8023 20.986) (width 0.25) (layer "F.Cu") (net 1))
 (segment (start 19.548 22.6292) (end 17.9048 20.986) (width 0.25) (layer "F.Cu") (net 1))
 (segment (start 15.2807 8.6752) (end 15.2807 7.1847) (width 0.25) (layer "F.Cu") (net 1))
 (segment (start 18.9535 23.9989) (end 19.548 23.4044) (width 0.25) (layer "F.Cu") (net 1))
 (segment (start 25.5404 12.2493) (end 26.2907 12.2493) (width 0.25) (layer "F.Cu") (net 1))
 (segment (start 21.1385 11.7368) (end 20.5007 11.7368) (width 0.25) (layer "F.Cu") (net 1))
 (segment (start 15.1335 18.3612) (end 14.0107 18.3612) (width 0.25) (layer "F.Cu") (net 1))
 (segment (start 28.6726 12.7707) (end 28.6726 11.7573) (width 0.25) (layer "F.Cu") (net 1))
 (segment (start 23.3157 14.7901) (end 23.3157 14.6243) (width 0.25) (layer "F.Cu") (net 1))
 (segment (start 21.1078 20.8022) (end 18.4557 18.1501) (width 0.25) (layer "F.Cu") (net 9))
 (segment (start 18.1857 28.0373) (end 21.1078 25.1152) (width 0.25) (layer "F.Cu") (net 9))
 (segment (start 21.1078 25.1152) (end 21.1078 20.8022) (width 0.25) (layer "F.Cu") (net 9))
 (segment (start 18.4557 18.1501) (end 18.4557 15.9118) (width 0.25) (layer "F.Cu") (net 9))
 (segment (start 13.0563 20.151) (end 13.6585 19.5488) (width 0.25) (layer "F.Cu") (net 7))
 (segment (start 9.112 6.0416) (end 9.112 19.4584) (width 0.25) (layer "F.Cu") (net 7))
 (segment (start 19.7257 16.6595) (end 20.8346 17.7684) (width 0.25) (layer "F.Cu") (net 7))
 (segment (start 13.847 21.6479) (end 10.5657 24.9292) (width 0.25) (layer "F.Cu") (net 7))
 (segment (start 14.0461 21.4488) (end 13.847 21.6479) (width 0.25) (layer "F.Cu") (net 7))
 (segment (start 8.7889 20.7873) (end 8.7889 23.3079) (width 0.25) (layer "F.Cu") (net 7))
 (segment (start 13.0563 20.8573) (end 13.0563 20.151) (width 0.25) (layer "F.Cu") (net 7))
 (segment (start 8.9284 25.2233) (end 10.5657 26.8606) (width 0.25) (layer "F.Cu") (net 7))
 (segment (start 8.7889 23.3079) (end 8.9284 23.4474) (width 0.25) (layer "F.Cu") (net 7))
 (segment (start 8.9284 23.4474) (end 8.9284 25.2233) (width 0.25) (layer "F.Cu") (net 7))
 (segment (start 19.7257 15.9118) (end 19.7257 16.6595) (width 0.25) (layer "F.Cu") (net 7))
 (segment (start 9.6149 19.9613) (end 8.7889 20.7873) (width 0.25) (layer "F.Cu") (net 7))
 (segment (start 9.112 19.4584) (end 9.6149 19.9613) (width 0.25) (layer "F.Cu") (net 7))
 (segment (start 13.847 21.6479) (end 13.0563 20.8573) (width 0.25) (layer "F.Cu") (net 7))
 (segment (start 10.5657 28.0373) (end 10.5657 26.8606) (width 0.25) (layer "F.Cu") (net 7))
 (segment (start 13.6585 19.5488) (end 14.0461 19.5488) (width 0.25) (layer "F.Cu") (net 7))
 (segment (start 10.5657 24.9292) (end 10.5657 26.8606) (width 0.25) (layer "F.Cu") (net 7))
 (via (at 20.8346 17.7684) (size 0.6) (drill 0.3) (layers "F.Cu" "B.Cu") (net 7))
 (segment (start 11.7424 26.8606) (end 20.8346 17.7684) (width 0.25) (layer "B.Cu") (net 7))
 (segment (start 10.5657 26.8606) (end 11.7424 26.8606) (width 0.25) (layer "B.Cu") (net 7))
 (segment (start 10.5657 28.0373) (end 10.5657 26.8606) (width 0.25) (layer "B.Cu") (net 7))
 (segment (start 19.4295 9.6079) (end 22.5845 9.6079) (width 0.25) (layer "F.Cu") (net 4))
 (segment (start 18.4557 10.9618) (end 18.4557 10.5817) (width 0.25) (layer "F.Cu") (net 4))
 (segment (start 23.3157 12.2493) (end 23.3157 11.4819) (width 0.25) (layer "F.Cu") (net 4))
 (segment (start 18.4557 10.5817) (end 19.4295 9.6079) (width 0.25) (layer "F.Cu") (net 4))
 (segment (start 22.5845 9.6079) (end 23.8871 10.9105) (width 0.25) (layer "F.Cu") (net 4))
 (segment (start 24.0483 10.7493) (end 24.1407 10.7493) (width 0.25) (layer "F.Cu") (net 4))
 (segment (start 23.3157 11.4819) (end 23.8871 10.9105) (width 0.25) (layer "F.Cu") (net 4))
 (segment (start 23.8871 10.9105) (end 24.0483 10.7493) (width 0.25) (layer "F.Cu") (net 4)))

